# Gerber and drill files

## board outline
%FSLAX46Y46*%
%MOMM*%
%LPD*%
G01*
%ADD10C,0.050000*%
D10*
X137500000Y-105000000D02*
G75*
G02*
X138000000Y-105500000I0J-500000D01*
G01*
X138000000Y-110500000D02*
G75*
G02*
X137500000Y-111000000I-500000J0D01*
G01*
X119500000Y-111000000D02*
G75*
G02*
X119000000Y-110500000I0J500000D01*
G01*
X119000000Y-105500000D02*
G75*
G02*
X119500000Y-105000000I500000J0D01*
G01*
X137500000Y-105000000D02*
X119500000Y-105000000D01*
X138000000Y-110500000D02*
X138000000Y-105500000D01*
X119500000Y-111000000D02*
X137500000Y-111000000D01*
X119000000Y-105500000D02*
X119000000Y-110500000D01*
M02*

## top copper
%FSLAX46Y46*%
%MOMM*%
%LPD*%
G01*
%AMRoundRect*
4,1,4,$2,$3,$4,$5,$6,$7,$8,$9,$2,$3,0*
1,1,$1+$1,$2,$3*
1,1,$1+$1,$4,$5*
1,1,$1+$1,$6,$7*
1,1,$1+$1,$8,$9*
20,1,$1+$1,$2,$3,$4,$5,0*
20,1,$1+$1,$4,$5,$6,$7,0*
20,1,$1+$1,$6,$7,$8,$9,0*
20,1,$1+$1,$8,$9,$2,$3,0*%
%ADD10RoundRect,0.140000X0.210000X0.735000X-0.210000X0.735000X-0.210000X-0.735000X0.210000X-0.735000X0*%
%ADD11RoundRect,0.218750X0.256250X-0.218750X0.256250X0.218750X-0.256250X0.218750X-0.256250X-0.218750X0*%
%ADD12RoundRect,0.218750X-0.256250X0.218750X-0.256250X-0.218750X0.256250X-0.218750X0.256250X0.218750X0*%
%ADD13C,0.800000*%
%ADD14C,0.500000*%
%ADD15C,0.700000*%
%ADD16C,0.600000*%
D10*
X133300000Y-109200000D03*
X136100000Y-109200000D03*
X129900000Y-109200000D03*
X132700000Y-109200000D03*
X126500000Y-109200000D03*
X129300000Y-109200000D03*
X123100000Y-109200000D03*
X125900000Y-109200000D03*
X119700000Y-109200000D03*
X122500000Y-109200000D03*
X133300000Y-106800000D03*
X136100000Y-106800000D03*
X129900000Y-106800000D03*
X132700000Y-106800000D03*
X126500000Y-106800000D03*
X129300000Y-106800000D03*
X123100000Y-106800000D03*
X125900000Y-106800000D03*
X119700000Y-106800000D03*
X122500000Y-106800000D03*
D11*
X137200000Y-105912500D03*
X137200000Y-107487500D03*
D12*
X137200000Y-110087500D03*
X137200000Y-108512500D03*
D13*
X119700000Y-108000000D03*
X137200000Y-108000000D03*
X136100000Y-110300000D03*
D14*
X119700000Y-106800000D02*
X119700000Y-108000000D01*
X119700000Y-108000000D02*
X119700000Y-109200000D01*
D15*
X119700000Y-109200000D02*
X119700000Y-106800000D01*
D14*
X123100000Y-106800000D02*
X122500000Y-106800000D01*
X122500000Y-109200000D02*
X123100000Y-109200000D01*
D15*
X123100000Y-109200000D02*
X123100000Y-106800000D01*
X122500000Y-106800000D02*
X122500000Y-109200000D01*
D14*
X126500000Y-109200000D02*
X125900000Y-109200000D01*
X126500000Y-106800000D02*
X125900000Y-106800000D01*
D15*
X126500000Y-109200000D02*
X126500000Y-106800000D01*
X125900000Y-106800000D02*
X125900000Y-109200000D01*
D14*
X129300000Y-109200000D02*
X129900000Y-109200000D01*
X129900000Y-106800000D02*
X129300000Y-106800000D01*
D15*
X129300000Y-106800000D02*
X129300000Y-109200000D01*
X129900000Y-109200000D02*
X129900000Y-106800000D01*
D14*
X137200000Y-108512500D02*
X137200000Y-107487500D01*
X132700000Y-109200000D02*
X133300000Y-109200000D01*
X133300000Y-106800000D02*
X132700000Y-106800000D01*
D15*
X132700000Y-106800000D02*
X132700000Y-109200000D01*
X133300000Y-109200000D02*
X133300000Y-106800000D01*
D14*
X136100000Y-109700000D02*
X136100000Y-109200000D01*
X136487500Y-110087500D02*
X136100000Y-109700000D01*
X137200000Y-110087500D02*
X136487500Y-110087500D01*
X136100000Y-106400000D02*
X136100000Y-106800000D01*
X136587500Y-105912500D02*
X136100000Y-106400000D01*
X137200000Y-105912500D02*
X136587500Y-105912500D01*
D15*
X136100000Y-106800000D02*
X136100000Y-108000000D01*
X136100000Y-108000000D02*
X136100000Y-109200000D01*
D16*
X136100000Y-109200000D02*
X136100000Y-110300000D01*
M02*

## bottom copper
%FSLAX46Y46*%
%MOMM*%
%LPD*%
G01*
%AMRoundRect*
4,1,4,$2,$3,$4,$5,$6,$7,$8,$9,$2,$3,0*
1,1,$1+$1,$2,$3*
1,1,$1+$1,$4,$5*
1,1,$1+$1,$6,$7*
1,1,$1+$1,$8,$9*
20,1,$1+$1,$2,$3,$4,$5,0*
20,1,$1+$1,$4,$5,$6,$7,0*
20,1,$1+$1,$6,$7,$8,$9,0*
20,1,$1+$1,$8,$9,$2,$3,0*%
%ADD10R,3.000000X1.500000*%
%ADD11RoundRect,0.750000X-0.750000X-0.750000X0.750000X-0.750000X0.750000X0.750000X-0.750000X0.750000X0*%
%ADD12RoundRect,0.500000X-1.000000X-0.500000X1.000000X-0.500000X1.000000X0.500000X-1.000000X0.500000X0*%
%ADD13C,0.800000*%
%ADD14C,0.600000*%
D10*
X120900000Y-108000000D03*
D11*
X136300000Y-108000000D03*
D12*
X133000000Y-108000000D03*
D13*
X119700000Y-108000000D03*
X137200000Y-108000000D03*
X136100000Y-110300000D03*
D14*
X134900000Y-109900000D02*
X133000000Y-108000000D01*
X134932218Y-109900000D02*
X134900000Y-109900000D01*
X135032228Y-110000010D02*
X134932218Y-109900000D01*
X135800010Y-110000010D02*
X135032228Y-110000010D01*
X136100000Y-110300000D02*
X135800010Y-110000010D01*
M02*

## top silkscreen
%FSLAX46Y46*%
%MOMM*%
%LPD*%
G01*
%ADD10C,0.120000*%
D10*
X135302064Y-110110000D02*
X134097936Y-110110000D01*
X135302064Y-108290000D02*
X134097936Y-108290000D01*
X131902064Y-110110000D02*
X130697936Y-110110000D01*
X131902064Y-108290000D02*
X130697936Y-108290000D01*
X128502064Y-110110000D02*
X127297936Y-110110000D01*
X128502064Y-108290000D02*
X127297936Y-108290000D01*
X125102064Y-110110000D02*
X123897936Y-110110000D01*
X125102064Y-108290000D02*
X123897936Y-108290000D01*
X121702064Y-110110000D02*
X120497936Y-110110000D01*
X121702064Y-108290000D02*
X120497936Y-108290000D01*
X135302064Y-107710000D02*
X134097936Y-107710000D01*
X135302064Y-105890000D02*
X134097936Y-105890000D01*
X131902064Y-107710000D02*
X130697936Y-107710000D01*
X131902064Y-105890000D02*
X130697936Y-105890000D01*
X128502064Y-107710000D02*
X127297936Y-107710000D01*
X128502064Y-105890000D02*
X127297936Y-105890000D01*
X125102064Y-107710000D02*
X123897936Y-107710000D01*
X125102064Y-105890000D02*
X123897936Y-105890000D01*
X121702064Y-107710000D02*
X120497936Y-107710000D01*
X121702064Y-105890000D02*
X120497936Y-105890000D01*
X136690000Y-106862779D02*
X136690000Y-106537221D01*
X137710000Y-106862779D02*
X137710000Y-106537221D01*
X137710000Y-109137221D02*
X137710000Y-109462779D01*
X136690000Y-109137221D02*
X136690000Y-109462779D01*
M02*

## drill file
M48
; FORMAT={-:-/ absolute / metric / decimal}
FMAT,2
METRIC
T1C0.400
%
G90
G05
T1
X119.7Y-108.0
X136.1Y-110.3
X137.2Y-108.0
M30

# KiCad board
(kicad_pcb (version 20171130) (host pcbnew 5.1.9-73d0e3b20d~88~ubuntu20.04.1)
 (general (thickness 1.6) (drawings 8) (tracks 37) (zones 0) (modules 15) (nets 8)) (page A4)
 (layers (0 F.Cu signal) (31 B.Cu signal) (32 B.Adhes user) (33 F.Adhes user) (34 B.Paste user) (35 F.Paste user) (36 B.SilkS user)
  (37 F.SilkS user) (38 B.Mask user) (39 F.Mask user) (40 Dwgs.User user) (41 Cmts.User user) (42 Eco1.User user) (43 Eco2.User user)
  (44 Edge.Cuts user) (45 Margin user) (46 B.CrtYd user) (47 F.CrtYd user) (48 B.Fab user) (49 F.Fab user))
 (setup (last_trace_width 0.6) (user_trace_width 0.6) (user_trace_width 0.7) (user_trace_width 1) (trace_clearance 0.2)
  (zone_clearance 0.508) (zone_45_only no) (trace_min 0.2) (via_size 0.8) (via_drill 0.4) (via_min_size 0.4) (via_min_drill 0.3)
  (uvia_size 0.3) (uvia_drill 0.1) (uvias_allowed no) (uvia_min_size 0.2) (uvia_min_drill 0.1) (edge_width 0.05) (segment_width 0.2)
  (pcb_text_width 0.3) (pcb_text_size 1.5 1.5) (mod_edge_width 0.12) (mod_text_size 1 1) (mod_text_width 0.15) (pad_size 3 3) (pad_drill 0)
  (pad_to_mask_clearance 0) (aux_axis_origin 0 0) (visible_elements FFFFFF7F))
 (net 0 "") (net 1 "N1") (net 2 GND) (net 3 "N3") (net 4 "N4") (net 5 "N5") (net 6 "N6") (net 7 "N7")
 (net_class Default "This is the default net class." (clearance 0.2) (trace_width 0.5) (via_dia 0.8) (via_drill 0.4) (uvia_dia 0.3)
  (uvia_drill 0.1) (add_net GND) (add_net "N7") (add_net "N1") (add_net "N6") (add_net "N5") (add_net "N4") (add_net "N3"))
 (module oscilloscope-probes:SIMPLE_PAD (layer B.Cu) (at 120.9 108 180)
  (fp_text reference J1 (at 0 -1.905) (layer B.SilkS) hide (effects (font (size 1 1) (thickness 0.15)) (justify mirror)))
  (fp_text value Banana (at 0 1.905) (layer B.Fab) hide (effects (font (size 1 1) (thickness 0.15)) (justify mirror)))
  (pad 1 smd rect (at 0 0 180) (size 3 1.5) (layers B.Cu B.Paste B.Mask) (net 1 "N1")))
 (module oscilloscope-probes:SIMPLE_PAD (layer B.Cu) (at 136.3 108)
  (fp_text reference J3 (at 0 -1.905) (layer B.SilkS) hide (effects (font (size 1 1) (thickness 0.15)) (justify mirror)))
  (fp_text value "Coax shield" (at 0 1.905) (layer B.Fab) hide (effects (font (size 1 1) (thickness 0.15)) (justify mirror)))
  (pad 1 smd roundrect (at 0 0) (size 3 3) (layers B.Cu B.Mask) (roundrect_rratio 0.25) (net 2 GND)))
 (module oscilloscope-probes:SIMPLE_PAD (layer B.Cu) (at 133 108)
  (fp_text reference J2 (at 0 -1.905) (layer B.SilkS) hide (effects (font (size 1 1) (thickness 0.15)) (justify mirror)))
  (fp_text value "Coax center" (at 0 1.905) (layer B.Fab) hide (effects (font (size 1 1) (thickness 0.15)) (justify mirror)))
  (pad 1 smd roundrect (at 0 0) (size 3 2) (layers B.Cu B.Mask) (roundrect_rratio 0.25) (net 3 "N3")))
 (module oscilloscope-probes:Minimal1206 (layer F.Cu) (at 134.7 109.2 180)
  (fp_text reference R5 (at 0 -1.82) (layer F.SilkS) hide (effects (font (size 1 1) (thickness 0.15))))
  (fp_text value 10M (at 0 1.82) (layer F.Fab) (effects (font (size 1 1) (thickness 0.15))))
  (fp_line (start -0.602064 -0.91) (end 0.602064 -0.91) (layer F.SilkS) (width 0.12))
  (fp_line (start -0.602064 0.91) (end 0.602064 0.91) (layer F.SilkS) (width 0.12))
  (pad 2 smd roundrect (at 1.4 0 180) (size 0.7 1.75) (layers F.Cu F.Paste F.Mask) (roundrect_rratio 0.2) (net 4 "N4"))
  (pad 1 smd roundrect (at -1.4 0 180) (size 0.7 1.75) (layers F.Cu F.Paste F.Mask) (roundrect_rratio 0.2) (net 3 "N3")))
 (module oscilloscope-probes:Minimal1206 (layer F.Cu) (at 131.3 109.2 180)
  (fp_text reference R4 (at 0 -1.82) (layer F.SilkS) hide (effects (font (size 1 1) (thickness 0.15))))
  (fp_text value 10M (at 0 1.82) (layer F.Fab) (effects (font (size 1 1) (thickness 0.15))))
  (fp_line (start -0.602064 -0.91) (end 0.602064 -0.91) (layer F.SilkS) (width 0.12))
  (fp_line (start -0.602064 0.91) (end 0.602064 0.91) (layer F.SilkS) (width 0.12))
  (pad 2 smd roundrect (at 1.4 0 180) (size 0.7 1.75) (layers F.Cu F.Paste F.Mask) (roundrect_rratio 0.2) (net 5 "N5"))
  (pad 1 smd roundrect (at -1.4 0 180) (size 0.7 1.75) (layers F.Cu F.Paste F.Mask) (roundrect_rratio 0.2) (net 4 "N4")))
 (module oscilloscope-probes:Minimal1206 (layer F.Cu) (at 127.9 109.2 180)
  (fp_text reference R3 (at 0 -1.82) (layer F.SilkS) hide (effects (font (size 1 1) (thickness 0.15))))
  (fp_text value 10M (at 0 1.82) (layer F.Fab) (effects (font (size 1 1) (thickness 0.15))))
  (fp_line (start -0.602064 -0.91) (end 0.602064 -0.91) (layer F.SilkS) (width 0.12))
  (fp_line (start -0.602064 0.91) (end 0.602064 0.91) (layer F.SilkS) (width 0.12))
  (pad 2 smd roundrect (at 1.4 0 180) (size 0.7 1.75) (layers F.Cu F.Paste F.Mask) (roundrect_rratio 0.2) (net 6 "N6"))
  (pad 1 smd roundrect (at -1.4 0 180) (size 0.7 1.75) (layers F.Cu F.Paste F.Mask) (roundrect_rratio 0.2) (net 5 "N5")))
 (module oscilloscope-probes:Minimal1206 (layer F.Cu) (at 124.5 109.2 180)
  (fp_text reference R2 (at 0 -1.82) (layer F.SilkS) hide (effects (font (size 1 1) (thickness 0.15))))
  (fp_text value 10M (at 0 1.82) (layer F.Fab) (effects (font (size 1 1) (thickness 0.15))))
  (fp_line (start -0.602064 -0.91) (end 0.602064 -0.91) (layer F.SilkS) (width 0.12))
  (fp_line (start -0.602064 0.91) (end 0.602064 0.91) (layer F.SilkS) (width 0.12))
  (pad 2 smd roundrect (at 1.4 0 180) (size 0.7 1.75) (layers F.Cu F.Paste F.Mask) (roundrect_rratio 0.2) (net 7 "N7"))
  (pad 1 smd roundrect (at -1.4 0 180) (size 0.7 1.75) (layers F.Cu F.Paste F.Mask) (roundrect_rratio 0.2) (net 6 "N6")))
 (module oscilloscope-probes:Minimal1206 (layer F.Cu) (at 121.1 109.2 180)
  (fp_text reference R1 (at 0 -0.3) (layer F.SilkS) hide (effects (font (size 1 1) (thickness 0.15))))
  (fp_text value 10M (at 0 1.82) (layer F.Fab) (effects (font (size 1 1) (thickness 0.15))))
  (fp_line (start -0.602064 -0.91) (end 0.602064 -0.91) (layer F.SilkS) (width 0.12))
  (fp_line (start -0.602064 0.91) (end 0.602064 0.91) (layer F.SilkS) (width 0.12))
  (pad 2 smd roundrect (at 1.4 0 180) (size 0.7 1.75) (layers F.Cu F.Paste F.Mask) (roundrect_rratio 0.2) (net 1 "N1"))
  (pad 1 smd roundrect (at -1.4 0 180) (size 0.7 1.75) (layers F.Cu F.Paste F.Mask) (roundrect_rratio 0.2) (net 7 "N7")))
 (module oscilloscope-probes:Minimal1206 (layer F.Cu) (at 134.7 106.8 180)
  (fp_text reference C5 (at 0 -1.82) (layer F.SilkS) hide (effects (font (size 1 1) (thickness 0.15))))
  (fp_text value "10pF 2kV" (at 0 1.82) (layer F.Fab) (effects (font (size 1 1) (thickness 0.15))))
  (fp_line (start -0.602064 -0.91) (end 0.602064 -0.91) (layer F.SilkS) (width 0.12))
  (fp_line (start -0.602064 0.91) (end 0.602064 0.91) (layer F.SilkS) (width 0.12))
  (pad 2 smd roundrect (at 1.4 0 180) (size 0.7 1.75) (layers F.Cu F.Paste F.Mask) (roundrect_rratio 0.2) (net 4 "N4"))
  (pad 1 smd roundrect (at -1.4 0 180) (size 0.7 1.75) (layers F.Cu F.Paste F.Mask) (roundrect_rratio 0.2) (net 3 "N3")))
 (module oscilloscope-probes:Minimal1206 (layer F.Cu) (at 131.3 106.8 180)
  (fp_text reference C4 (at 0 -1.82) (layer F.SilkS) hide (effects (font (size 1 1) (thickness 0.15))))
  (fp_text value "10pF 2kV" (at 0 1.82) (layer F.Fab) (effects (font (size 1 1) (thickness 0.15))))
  (fp_line (start -0.602064 -0.91) (end 0.602064 -0.91) (layer F.SilkS) (width 0.12))
  (fp_line (start -0.602064 0.91) (end 0.602064 0.91) (layer F.SilkS) (width 0.12))
  (pad 2 smd roundrect (at 1.4 0 180) (size 0.7 1.75) (layers F.Cu F.Paste F.Mask) (roundrect_rratio 0.2) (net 5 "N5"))
  (pad 1 smd roundrect (at -1.4 0 180) (size 0.7 1.75) (layers F.Cu F.Paste F.Mask) (roundrect_rratio 0.2) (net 4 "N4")))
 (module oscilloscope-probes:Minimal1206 (layer F.Cu) (at 127.9 106.8 180)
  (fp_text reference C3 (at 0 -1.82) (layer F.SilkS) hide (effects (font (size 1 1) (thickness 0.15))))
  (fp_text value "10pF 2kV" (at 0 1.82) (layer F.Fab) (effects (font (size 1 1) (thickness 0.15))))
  (fp_line (start -0.602064 -0.91) (end 0.602064 -0.91) (layer F.SilkS) (width 0.12))
  (fp_line (start -0.602064 0.91) (end 0.602064 0.91) (layer F.SilkS) (width 0.12))
  (pad 2 smd roundrect (at 1.4 0 180) (size 0.7 1.75) (layers F.Cu F.Paste F.Mask) (roundrect_rratio 0.2) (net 6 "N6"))
  (pad 1 smd roundrect (at -1.4 0 180) (size 0.7 1.75) (layers F.Cu F.Paste F.Mask) (roundrect_rratio 0.2) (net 5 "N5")))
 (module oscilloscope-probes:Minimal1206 (layer F.Cu) (at 124.5 106.8 180)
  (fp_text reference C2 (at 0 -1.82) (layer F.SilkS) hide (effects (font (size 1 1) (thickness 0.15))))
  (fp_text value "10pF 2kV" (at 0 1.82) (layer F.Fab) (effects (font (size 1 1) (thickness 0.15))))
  (fp_line (start -0.602064 -0.91) (end 0.602064 -0.91) (layer F.SilkS) (width 0.12))
  (fp_line (start -0.602064 0.91) (end 0.602064 0.91) (layer F.SilkS) (width 0.12))
  (pad 2 smd roundrect (at 1.4 0 180) (size 0.7 1.75) (layers F.Cu F.Paste F.Mask) (roundrect_rratio 0.2) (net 7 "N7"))
  (pad 1 smd roundrect (at -1.4 0 180) (size 0.7 1.75) (layers F.Cu F.Paste F.Mask) (roundrect_rratio 0.2) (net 6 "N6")))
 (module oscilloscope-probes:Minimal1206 (layer F.Cu) (at 121.1 106.8 180)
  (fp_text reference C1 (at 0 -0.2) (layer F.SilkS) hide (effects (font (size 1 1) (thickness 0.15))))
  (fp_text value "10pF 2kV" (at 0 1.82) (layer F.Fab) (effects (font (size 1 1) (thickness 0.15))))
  (fp_line (start -0.602064 -0.91) (end 0.602064 -0.91) (layer F.SilkS) (width 0.12))
  (fp_line (start -0.602064 0.91) (end 0.602064 0.91) (layer F.SilkS) (width 0.12))
  (pad 2 smd roundrect (at 1.4 0 180) (size 0.7 1.75) (layers F.Cu F.Paste F.Mask) (roundrect_rratio 0.2) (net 1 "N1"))
  (pad 1 smd roundrect (at -1.4 0 180) (size 0.7 1.75) (layers F.Cu F.Paste F.Mask) (roundrect_rratio 0.2) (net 7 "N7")))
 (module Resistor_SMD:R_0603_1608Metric (layer F.Cu) (at 137.2 106.7 90)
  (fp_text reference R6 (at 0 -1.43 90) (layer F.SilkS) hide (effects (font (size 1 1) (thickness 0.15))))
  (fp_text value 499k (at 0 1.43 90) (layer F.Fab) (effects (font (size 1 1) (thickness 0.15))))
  (fp_line (start -0.162779 -0.51) (end 0.162779 -0.51) (layer F.SilkS) (width 0.12))
  (fp_line (start -0.162779 0.51) (end 0.162779 0.51) (layer F.SilkS) (width 0.12))
  (pad 2 smd roundrect (at 0.7875 0 90) (size 0.875 0.95) (layers F.Cu F.Paste F.Mask) (roundrect_rratio 0.25) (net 3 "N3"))
  (pad 1 smd roundrect (at -0.7875 0 90) (size 0.875 0.95) (layers F.Cu F.Paste F.Mask) (roundrect_rratio 0.25) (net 2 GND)))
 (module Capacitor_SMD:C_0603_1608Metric (layer F.Cu) (at 137.2 109.3 270)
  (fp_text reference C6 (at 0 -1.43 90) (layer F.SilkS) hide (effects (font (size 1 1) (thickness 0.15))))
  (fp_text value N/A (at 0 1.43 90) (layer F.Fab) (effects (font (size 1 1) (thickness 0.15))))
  (fp_line (start -0.162779 -0.51) (end 0.162779 -0.51) (layer F.SilkS) (width 0.12))
  (fp_line (start -0.162779 0.51) (end 0.162779 0.51) (layer F.SilkS) (width 0.12))
  (pad 2 smd roundrect (at 0.7875 0 270) (size 0.875 0.95) (layers F.Cu F.Paste F.Mask) (roundrect_rratio 0.25) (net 3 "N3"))
  (pad 1 smd roundrect (at -0.7875 0 270) (size 0.875 0.95) (layers F.Cu F.Paste F.Mask) (roundrect_rratio 0.25) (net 2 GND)))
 (gr_arc (start 137.5 105.5) (end 138 105.5) (angle -90) (layer Edge.Cuts) (width 0.05))
 (gr_arc (start 137.5 110.5) (end 137.5 111) (angle -90) (layer Edge.Cuts) (width 0.05))
 (gr_arc (start 119.5 110.5) (end 119 110.5) (angle -90) (layer Edge.Cuts) (width 0.05))
 (gr_arc (start 119.5 105.5) (end 119.5 105) (angle -90) (layer Edge.Cuts) (width 0.05))
 (gr_line (start 137.5 105) (end 119.5 105) (layer Edge.Cuts) (width 0.05))
 (gr_line (start 138 110.5) (end 138 105.5) (layer Edge.Cuts) (width 0.05))
 (gr_line (start 119.5 111) (end 137.5 111) (layer Edge.Cuts) (width 0.05))
 (gr_line (start 119 105.5) (end 119 110.5) (layer Edge.Cuts) (width 0.05))
 (via (at 119.7 108) (size 0.8) (drill 0.4) (layers F.Cu B.Cu) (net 1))
 (segment (start 119.7 106.8) (end 119.7 108) (width 0.5) (layer F.Cu) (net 1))
 (segment (start 119.7 108) (end 119.7 109.2) (width 0.5) (layer F.Cu) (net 1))
 (segment (start 119.7 109.2) (end 119.7 106.8) (width 0.7) (layer F.Cu) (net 1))
 (segment (start 123.1 106.8) (end 122.5 106.8) (width 0.5) (layer F.Cu) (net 7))
 (segment (start 122.5 109.2) (end 123.1 109.2) (width 0.5) (layer F.Cu) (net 7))
 (segment (start 123.1 109.2) (end 123.1 106.8) (width 0.7) (layer F.Cu) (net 7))
 (segment (start 122.5 106.8) (end 122.5 109.2) (width 0.7) (layer F.Cu) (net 7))
 (segment (start 126.5 109.2) (end 125.9 109.2) (width 0.5) (layer F.Cu) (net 6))
 (segment (start 126.5 106.8) (end 125.9 106.8) (width 0.5) (layer F.Cu) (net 6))
 (segment (start 126.5 109.2) (end 126.5 106.8) (width 0.7) (layer F.Cu) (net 6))
 (segment (start 125.9 106.8) (end 125.9 109.2) (width 0.7) (layer F.Cu) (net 6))
 (segment (start 129.3 109.2) (end 129.9 109.2) (width 0.5) (layer F.Cu) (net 5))
 (segment (start 129.9 106.8) (end 129.3 106.8) (width 0.5) (layer F.Cu) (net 5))
 (segment (start 129.3 106.8) (end 129.3 109.2) (width 0.7) (layer F.Cu) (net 5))
 (segment (start 129.9 109.2) (end 129.9 106.8) (width 0.7) (layer F.Cu) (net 5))
 (segment (start 137.2 108.5125) (end 137.2 107.4875) (width 0.5) (layer F.Cu) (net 2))
 (via (at 137.2 108) (size 0.8) (drill 0.4) (layers F.Cu B.Cu) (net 2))
 (segment (start 132.7 109.2) (end 133.3 109.2) (width 0.5) (layer F.Cu) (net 4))
 (segment (start 133.3 106.8) (end 132.7 106.8) (width 0.5) (layer F.Cu) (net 4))
 (segment (start 132.7 106.8) (end 132.7 109.2) (width 0.7) (layer F.Cu) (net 4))
 (segment (start 133.3 109.2) (end 133.3 106.8) (width 0.7) (layer F.Cu) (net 4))
 (segment (start 136.1 109.7) (end 136.1 109.2) (width 0.5) (layer F.Cu) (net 3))
 (segment (start 136.4875 110.0875) (end 136.1 109.7) (width 0.5) (layer F.Cu) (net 3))
 (segment (start 137.2 110.0875) (end 136.4875 110.0875) (width 0.5) (layer F.Cu) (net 3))
 (segment (start 136.1 106.4) (end 136.1 106.8) (width 0.5) (layer F.Cu) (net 3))
 (segment (start 136.5875 105.9125) (end 136.1 106.4) (width 0.5) (layer F.Cu) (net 3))
 (segment (start 137.2 105.9125) (end 136.5875 105.9125) (width 0.5) (layer F.Cu) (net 3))
 (segment (start 136.1 106.8) (end 136.1 108) (width 0.7) (layer F.Cu) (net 3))
 (segment (start 136.1 108) (end 136.1 109.2) (width 0.7) (layer F.Cu) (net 3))
 (via (at 136.1 110.3) (size 0.8) (drill 0.4) (layers F.Cu B.Cu) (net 3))
 (segment (start 136.1 109.2) (end 136.1 110.3) (width 0.6) (layer F.Cu) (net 3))
 (segment (start 134.9 109.9) (end 133 108) (width 0.6) (layer B.Cu) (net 3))
 (segment (start 134.932218 109.9) (end 134.9 109.9) (width 0.6) (layer B.Cu) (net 3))
 (segment (start 135.032228 110.00001) (end 134.932218 109.9) (width 0.6) (layer B.Cu) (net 3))
 (segment (start 135.80001 110.00001) (end 135.032228 110.00001) (width 0.6) (layer B.Cu) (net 3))
 (segment (start 136.1 110.3) (end 135.80001 110.00001) (width 0.6) (layer B.Cu) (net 3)))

